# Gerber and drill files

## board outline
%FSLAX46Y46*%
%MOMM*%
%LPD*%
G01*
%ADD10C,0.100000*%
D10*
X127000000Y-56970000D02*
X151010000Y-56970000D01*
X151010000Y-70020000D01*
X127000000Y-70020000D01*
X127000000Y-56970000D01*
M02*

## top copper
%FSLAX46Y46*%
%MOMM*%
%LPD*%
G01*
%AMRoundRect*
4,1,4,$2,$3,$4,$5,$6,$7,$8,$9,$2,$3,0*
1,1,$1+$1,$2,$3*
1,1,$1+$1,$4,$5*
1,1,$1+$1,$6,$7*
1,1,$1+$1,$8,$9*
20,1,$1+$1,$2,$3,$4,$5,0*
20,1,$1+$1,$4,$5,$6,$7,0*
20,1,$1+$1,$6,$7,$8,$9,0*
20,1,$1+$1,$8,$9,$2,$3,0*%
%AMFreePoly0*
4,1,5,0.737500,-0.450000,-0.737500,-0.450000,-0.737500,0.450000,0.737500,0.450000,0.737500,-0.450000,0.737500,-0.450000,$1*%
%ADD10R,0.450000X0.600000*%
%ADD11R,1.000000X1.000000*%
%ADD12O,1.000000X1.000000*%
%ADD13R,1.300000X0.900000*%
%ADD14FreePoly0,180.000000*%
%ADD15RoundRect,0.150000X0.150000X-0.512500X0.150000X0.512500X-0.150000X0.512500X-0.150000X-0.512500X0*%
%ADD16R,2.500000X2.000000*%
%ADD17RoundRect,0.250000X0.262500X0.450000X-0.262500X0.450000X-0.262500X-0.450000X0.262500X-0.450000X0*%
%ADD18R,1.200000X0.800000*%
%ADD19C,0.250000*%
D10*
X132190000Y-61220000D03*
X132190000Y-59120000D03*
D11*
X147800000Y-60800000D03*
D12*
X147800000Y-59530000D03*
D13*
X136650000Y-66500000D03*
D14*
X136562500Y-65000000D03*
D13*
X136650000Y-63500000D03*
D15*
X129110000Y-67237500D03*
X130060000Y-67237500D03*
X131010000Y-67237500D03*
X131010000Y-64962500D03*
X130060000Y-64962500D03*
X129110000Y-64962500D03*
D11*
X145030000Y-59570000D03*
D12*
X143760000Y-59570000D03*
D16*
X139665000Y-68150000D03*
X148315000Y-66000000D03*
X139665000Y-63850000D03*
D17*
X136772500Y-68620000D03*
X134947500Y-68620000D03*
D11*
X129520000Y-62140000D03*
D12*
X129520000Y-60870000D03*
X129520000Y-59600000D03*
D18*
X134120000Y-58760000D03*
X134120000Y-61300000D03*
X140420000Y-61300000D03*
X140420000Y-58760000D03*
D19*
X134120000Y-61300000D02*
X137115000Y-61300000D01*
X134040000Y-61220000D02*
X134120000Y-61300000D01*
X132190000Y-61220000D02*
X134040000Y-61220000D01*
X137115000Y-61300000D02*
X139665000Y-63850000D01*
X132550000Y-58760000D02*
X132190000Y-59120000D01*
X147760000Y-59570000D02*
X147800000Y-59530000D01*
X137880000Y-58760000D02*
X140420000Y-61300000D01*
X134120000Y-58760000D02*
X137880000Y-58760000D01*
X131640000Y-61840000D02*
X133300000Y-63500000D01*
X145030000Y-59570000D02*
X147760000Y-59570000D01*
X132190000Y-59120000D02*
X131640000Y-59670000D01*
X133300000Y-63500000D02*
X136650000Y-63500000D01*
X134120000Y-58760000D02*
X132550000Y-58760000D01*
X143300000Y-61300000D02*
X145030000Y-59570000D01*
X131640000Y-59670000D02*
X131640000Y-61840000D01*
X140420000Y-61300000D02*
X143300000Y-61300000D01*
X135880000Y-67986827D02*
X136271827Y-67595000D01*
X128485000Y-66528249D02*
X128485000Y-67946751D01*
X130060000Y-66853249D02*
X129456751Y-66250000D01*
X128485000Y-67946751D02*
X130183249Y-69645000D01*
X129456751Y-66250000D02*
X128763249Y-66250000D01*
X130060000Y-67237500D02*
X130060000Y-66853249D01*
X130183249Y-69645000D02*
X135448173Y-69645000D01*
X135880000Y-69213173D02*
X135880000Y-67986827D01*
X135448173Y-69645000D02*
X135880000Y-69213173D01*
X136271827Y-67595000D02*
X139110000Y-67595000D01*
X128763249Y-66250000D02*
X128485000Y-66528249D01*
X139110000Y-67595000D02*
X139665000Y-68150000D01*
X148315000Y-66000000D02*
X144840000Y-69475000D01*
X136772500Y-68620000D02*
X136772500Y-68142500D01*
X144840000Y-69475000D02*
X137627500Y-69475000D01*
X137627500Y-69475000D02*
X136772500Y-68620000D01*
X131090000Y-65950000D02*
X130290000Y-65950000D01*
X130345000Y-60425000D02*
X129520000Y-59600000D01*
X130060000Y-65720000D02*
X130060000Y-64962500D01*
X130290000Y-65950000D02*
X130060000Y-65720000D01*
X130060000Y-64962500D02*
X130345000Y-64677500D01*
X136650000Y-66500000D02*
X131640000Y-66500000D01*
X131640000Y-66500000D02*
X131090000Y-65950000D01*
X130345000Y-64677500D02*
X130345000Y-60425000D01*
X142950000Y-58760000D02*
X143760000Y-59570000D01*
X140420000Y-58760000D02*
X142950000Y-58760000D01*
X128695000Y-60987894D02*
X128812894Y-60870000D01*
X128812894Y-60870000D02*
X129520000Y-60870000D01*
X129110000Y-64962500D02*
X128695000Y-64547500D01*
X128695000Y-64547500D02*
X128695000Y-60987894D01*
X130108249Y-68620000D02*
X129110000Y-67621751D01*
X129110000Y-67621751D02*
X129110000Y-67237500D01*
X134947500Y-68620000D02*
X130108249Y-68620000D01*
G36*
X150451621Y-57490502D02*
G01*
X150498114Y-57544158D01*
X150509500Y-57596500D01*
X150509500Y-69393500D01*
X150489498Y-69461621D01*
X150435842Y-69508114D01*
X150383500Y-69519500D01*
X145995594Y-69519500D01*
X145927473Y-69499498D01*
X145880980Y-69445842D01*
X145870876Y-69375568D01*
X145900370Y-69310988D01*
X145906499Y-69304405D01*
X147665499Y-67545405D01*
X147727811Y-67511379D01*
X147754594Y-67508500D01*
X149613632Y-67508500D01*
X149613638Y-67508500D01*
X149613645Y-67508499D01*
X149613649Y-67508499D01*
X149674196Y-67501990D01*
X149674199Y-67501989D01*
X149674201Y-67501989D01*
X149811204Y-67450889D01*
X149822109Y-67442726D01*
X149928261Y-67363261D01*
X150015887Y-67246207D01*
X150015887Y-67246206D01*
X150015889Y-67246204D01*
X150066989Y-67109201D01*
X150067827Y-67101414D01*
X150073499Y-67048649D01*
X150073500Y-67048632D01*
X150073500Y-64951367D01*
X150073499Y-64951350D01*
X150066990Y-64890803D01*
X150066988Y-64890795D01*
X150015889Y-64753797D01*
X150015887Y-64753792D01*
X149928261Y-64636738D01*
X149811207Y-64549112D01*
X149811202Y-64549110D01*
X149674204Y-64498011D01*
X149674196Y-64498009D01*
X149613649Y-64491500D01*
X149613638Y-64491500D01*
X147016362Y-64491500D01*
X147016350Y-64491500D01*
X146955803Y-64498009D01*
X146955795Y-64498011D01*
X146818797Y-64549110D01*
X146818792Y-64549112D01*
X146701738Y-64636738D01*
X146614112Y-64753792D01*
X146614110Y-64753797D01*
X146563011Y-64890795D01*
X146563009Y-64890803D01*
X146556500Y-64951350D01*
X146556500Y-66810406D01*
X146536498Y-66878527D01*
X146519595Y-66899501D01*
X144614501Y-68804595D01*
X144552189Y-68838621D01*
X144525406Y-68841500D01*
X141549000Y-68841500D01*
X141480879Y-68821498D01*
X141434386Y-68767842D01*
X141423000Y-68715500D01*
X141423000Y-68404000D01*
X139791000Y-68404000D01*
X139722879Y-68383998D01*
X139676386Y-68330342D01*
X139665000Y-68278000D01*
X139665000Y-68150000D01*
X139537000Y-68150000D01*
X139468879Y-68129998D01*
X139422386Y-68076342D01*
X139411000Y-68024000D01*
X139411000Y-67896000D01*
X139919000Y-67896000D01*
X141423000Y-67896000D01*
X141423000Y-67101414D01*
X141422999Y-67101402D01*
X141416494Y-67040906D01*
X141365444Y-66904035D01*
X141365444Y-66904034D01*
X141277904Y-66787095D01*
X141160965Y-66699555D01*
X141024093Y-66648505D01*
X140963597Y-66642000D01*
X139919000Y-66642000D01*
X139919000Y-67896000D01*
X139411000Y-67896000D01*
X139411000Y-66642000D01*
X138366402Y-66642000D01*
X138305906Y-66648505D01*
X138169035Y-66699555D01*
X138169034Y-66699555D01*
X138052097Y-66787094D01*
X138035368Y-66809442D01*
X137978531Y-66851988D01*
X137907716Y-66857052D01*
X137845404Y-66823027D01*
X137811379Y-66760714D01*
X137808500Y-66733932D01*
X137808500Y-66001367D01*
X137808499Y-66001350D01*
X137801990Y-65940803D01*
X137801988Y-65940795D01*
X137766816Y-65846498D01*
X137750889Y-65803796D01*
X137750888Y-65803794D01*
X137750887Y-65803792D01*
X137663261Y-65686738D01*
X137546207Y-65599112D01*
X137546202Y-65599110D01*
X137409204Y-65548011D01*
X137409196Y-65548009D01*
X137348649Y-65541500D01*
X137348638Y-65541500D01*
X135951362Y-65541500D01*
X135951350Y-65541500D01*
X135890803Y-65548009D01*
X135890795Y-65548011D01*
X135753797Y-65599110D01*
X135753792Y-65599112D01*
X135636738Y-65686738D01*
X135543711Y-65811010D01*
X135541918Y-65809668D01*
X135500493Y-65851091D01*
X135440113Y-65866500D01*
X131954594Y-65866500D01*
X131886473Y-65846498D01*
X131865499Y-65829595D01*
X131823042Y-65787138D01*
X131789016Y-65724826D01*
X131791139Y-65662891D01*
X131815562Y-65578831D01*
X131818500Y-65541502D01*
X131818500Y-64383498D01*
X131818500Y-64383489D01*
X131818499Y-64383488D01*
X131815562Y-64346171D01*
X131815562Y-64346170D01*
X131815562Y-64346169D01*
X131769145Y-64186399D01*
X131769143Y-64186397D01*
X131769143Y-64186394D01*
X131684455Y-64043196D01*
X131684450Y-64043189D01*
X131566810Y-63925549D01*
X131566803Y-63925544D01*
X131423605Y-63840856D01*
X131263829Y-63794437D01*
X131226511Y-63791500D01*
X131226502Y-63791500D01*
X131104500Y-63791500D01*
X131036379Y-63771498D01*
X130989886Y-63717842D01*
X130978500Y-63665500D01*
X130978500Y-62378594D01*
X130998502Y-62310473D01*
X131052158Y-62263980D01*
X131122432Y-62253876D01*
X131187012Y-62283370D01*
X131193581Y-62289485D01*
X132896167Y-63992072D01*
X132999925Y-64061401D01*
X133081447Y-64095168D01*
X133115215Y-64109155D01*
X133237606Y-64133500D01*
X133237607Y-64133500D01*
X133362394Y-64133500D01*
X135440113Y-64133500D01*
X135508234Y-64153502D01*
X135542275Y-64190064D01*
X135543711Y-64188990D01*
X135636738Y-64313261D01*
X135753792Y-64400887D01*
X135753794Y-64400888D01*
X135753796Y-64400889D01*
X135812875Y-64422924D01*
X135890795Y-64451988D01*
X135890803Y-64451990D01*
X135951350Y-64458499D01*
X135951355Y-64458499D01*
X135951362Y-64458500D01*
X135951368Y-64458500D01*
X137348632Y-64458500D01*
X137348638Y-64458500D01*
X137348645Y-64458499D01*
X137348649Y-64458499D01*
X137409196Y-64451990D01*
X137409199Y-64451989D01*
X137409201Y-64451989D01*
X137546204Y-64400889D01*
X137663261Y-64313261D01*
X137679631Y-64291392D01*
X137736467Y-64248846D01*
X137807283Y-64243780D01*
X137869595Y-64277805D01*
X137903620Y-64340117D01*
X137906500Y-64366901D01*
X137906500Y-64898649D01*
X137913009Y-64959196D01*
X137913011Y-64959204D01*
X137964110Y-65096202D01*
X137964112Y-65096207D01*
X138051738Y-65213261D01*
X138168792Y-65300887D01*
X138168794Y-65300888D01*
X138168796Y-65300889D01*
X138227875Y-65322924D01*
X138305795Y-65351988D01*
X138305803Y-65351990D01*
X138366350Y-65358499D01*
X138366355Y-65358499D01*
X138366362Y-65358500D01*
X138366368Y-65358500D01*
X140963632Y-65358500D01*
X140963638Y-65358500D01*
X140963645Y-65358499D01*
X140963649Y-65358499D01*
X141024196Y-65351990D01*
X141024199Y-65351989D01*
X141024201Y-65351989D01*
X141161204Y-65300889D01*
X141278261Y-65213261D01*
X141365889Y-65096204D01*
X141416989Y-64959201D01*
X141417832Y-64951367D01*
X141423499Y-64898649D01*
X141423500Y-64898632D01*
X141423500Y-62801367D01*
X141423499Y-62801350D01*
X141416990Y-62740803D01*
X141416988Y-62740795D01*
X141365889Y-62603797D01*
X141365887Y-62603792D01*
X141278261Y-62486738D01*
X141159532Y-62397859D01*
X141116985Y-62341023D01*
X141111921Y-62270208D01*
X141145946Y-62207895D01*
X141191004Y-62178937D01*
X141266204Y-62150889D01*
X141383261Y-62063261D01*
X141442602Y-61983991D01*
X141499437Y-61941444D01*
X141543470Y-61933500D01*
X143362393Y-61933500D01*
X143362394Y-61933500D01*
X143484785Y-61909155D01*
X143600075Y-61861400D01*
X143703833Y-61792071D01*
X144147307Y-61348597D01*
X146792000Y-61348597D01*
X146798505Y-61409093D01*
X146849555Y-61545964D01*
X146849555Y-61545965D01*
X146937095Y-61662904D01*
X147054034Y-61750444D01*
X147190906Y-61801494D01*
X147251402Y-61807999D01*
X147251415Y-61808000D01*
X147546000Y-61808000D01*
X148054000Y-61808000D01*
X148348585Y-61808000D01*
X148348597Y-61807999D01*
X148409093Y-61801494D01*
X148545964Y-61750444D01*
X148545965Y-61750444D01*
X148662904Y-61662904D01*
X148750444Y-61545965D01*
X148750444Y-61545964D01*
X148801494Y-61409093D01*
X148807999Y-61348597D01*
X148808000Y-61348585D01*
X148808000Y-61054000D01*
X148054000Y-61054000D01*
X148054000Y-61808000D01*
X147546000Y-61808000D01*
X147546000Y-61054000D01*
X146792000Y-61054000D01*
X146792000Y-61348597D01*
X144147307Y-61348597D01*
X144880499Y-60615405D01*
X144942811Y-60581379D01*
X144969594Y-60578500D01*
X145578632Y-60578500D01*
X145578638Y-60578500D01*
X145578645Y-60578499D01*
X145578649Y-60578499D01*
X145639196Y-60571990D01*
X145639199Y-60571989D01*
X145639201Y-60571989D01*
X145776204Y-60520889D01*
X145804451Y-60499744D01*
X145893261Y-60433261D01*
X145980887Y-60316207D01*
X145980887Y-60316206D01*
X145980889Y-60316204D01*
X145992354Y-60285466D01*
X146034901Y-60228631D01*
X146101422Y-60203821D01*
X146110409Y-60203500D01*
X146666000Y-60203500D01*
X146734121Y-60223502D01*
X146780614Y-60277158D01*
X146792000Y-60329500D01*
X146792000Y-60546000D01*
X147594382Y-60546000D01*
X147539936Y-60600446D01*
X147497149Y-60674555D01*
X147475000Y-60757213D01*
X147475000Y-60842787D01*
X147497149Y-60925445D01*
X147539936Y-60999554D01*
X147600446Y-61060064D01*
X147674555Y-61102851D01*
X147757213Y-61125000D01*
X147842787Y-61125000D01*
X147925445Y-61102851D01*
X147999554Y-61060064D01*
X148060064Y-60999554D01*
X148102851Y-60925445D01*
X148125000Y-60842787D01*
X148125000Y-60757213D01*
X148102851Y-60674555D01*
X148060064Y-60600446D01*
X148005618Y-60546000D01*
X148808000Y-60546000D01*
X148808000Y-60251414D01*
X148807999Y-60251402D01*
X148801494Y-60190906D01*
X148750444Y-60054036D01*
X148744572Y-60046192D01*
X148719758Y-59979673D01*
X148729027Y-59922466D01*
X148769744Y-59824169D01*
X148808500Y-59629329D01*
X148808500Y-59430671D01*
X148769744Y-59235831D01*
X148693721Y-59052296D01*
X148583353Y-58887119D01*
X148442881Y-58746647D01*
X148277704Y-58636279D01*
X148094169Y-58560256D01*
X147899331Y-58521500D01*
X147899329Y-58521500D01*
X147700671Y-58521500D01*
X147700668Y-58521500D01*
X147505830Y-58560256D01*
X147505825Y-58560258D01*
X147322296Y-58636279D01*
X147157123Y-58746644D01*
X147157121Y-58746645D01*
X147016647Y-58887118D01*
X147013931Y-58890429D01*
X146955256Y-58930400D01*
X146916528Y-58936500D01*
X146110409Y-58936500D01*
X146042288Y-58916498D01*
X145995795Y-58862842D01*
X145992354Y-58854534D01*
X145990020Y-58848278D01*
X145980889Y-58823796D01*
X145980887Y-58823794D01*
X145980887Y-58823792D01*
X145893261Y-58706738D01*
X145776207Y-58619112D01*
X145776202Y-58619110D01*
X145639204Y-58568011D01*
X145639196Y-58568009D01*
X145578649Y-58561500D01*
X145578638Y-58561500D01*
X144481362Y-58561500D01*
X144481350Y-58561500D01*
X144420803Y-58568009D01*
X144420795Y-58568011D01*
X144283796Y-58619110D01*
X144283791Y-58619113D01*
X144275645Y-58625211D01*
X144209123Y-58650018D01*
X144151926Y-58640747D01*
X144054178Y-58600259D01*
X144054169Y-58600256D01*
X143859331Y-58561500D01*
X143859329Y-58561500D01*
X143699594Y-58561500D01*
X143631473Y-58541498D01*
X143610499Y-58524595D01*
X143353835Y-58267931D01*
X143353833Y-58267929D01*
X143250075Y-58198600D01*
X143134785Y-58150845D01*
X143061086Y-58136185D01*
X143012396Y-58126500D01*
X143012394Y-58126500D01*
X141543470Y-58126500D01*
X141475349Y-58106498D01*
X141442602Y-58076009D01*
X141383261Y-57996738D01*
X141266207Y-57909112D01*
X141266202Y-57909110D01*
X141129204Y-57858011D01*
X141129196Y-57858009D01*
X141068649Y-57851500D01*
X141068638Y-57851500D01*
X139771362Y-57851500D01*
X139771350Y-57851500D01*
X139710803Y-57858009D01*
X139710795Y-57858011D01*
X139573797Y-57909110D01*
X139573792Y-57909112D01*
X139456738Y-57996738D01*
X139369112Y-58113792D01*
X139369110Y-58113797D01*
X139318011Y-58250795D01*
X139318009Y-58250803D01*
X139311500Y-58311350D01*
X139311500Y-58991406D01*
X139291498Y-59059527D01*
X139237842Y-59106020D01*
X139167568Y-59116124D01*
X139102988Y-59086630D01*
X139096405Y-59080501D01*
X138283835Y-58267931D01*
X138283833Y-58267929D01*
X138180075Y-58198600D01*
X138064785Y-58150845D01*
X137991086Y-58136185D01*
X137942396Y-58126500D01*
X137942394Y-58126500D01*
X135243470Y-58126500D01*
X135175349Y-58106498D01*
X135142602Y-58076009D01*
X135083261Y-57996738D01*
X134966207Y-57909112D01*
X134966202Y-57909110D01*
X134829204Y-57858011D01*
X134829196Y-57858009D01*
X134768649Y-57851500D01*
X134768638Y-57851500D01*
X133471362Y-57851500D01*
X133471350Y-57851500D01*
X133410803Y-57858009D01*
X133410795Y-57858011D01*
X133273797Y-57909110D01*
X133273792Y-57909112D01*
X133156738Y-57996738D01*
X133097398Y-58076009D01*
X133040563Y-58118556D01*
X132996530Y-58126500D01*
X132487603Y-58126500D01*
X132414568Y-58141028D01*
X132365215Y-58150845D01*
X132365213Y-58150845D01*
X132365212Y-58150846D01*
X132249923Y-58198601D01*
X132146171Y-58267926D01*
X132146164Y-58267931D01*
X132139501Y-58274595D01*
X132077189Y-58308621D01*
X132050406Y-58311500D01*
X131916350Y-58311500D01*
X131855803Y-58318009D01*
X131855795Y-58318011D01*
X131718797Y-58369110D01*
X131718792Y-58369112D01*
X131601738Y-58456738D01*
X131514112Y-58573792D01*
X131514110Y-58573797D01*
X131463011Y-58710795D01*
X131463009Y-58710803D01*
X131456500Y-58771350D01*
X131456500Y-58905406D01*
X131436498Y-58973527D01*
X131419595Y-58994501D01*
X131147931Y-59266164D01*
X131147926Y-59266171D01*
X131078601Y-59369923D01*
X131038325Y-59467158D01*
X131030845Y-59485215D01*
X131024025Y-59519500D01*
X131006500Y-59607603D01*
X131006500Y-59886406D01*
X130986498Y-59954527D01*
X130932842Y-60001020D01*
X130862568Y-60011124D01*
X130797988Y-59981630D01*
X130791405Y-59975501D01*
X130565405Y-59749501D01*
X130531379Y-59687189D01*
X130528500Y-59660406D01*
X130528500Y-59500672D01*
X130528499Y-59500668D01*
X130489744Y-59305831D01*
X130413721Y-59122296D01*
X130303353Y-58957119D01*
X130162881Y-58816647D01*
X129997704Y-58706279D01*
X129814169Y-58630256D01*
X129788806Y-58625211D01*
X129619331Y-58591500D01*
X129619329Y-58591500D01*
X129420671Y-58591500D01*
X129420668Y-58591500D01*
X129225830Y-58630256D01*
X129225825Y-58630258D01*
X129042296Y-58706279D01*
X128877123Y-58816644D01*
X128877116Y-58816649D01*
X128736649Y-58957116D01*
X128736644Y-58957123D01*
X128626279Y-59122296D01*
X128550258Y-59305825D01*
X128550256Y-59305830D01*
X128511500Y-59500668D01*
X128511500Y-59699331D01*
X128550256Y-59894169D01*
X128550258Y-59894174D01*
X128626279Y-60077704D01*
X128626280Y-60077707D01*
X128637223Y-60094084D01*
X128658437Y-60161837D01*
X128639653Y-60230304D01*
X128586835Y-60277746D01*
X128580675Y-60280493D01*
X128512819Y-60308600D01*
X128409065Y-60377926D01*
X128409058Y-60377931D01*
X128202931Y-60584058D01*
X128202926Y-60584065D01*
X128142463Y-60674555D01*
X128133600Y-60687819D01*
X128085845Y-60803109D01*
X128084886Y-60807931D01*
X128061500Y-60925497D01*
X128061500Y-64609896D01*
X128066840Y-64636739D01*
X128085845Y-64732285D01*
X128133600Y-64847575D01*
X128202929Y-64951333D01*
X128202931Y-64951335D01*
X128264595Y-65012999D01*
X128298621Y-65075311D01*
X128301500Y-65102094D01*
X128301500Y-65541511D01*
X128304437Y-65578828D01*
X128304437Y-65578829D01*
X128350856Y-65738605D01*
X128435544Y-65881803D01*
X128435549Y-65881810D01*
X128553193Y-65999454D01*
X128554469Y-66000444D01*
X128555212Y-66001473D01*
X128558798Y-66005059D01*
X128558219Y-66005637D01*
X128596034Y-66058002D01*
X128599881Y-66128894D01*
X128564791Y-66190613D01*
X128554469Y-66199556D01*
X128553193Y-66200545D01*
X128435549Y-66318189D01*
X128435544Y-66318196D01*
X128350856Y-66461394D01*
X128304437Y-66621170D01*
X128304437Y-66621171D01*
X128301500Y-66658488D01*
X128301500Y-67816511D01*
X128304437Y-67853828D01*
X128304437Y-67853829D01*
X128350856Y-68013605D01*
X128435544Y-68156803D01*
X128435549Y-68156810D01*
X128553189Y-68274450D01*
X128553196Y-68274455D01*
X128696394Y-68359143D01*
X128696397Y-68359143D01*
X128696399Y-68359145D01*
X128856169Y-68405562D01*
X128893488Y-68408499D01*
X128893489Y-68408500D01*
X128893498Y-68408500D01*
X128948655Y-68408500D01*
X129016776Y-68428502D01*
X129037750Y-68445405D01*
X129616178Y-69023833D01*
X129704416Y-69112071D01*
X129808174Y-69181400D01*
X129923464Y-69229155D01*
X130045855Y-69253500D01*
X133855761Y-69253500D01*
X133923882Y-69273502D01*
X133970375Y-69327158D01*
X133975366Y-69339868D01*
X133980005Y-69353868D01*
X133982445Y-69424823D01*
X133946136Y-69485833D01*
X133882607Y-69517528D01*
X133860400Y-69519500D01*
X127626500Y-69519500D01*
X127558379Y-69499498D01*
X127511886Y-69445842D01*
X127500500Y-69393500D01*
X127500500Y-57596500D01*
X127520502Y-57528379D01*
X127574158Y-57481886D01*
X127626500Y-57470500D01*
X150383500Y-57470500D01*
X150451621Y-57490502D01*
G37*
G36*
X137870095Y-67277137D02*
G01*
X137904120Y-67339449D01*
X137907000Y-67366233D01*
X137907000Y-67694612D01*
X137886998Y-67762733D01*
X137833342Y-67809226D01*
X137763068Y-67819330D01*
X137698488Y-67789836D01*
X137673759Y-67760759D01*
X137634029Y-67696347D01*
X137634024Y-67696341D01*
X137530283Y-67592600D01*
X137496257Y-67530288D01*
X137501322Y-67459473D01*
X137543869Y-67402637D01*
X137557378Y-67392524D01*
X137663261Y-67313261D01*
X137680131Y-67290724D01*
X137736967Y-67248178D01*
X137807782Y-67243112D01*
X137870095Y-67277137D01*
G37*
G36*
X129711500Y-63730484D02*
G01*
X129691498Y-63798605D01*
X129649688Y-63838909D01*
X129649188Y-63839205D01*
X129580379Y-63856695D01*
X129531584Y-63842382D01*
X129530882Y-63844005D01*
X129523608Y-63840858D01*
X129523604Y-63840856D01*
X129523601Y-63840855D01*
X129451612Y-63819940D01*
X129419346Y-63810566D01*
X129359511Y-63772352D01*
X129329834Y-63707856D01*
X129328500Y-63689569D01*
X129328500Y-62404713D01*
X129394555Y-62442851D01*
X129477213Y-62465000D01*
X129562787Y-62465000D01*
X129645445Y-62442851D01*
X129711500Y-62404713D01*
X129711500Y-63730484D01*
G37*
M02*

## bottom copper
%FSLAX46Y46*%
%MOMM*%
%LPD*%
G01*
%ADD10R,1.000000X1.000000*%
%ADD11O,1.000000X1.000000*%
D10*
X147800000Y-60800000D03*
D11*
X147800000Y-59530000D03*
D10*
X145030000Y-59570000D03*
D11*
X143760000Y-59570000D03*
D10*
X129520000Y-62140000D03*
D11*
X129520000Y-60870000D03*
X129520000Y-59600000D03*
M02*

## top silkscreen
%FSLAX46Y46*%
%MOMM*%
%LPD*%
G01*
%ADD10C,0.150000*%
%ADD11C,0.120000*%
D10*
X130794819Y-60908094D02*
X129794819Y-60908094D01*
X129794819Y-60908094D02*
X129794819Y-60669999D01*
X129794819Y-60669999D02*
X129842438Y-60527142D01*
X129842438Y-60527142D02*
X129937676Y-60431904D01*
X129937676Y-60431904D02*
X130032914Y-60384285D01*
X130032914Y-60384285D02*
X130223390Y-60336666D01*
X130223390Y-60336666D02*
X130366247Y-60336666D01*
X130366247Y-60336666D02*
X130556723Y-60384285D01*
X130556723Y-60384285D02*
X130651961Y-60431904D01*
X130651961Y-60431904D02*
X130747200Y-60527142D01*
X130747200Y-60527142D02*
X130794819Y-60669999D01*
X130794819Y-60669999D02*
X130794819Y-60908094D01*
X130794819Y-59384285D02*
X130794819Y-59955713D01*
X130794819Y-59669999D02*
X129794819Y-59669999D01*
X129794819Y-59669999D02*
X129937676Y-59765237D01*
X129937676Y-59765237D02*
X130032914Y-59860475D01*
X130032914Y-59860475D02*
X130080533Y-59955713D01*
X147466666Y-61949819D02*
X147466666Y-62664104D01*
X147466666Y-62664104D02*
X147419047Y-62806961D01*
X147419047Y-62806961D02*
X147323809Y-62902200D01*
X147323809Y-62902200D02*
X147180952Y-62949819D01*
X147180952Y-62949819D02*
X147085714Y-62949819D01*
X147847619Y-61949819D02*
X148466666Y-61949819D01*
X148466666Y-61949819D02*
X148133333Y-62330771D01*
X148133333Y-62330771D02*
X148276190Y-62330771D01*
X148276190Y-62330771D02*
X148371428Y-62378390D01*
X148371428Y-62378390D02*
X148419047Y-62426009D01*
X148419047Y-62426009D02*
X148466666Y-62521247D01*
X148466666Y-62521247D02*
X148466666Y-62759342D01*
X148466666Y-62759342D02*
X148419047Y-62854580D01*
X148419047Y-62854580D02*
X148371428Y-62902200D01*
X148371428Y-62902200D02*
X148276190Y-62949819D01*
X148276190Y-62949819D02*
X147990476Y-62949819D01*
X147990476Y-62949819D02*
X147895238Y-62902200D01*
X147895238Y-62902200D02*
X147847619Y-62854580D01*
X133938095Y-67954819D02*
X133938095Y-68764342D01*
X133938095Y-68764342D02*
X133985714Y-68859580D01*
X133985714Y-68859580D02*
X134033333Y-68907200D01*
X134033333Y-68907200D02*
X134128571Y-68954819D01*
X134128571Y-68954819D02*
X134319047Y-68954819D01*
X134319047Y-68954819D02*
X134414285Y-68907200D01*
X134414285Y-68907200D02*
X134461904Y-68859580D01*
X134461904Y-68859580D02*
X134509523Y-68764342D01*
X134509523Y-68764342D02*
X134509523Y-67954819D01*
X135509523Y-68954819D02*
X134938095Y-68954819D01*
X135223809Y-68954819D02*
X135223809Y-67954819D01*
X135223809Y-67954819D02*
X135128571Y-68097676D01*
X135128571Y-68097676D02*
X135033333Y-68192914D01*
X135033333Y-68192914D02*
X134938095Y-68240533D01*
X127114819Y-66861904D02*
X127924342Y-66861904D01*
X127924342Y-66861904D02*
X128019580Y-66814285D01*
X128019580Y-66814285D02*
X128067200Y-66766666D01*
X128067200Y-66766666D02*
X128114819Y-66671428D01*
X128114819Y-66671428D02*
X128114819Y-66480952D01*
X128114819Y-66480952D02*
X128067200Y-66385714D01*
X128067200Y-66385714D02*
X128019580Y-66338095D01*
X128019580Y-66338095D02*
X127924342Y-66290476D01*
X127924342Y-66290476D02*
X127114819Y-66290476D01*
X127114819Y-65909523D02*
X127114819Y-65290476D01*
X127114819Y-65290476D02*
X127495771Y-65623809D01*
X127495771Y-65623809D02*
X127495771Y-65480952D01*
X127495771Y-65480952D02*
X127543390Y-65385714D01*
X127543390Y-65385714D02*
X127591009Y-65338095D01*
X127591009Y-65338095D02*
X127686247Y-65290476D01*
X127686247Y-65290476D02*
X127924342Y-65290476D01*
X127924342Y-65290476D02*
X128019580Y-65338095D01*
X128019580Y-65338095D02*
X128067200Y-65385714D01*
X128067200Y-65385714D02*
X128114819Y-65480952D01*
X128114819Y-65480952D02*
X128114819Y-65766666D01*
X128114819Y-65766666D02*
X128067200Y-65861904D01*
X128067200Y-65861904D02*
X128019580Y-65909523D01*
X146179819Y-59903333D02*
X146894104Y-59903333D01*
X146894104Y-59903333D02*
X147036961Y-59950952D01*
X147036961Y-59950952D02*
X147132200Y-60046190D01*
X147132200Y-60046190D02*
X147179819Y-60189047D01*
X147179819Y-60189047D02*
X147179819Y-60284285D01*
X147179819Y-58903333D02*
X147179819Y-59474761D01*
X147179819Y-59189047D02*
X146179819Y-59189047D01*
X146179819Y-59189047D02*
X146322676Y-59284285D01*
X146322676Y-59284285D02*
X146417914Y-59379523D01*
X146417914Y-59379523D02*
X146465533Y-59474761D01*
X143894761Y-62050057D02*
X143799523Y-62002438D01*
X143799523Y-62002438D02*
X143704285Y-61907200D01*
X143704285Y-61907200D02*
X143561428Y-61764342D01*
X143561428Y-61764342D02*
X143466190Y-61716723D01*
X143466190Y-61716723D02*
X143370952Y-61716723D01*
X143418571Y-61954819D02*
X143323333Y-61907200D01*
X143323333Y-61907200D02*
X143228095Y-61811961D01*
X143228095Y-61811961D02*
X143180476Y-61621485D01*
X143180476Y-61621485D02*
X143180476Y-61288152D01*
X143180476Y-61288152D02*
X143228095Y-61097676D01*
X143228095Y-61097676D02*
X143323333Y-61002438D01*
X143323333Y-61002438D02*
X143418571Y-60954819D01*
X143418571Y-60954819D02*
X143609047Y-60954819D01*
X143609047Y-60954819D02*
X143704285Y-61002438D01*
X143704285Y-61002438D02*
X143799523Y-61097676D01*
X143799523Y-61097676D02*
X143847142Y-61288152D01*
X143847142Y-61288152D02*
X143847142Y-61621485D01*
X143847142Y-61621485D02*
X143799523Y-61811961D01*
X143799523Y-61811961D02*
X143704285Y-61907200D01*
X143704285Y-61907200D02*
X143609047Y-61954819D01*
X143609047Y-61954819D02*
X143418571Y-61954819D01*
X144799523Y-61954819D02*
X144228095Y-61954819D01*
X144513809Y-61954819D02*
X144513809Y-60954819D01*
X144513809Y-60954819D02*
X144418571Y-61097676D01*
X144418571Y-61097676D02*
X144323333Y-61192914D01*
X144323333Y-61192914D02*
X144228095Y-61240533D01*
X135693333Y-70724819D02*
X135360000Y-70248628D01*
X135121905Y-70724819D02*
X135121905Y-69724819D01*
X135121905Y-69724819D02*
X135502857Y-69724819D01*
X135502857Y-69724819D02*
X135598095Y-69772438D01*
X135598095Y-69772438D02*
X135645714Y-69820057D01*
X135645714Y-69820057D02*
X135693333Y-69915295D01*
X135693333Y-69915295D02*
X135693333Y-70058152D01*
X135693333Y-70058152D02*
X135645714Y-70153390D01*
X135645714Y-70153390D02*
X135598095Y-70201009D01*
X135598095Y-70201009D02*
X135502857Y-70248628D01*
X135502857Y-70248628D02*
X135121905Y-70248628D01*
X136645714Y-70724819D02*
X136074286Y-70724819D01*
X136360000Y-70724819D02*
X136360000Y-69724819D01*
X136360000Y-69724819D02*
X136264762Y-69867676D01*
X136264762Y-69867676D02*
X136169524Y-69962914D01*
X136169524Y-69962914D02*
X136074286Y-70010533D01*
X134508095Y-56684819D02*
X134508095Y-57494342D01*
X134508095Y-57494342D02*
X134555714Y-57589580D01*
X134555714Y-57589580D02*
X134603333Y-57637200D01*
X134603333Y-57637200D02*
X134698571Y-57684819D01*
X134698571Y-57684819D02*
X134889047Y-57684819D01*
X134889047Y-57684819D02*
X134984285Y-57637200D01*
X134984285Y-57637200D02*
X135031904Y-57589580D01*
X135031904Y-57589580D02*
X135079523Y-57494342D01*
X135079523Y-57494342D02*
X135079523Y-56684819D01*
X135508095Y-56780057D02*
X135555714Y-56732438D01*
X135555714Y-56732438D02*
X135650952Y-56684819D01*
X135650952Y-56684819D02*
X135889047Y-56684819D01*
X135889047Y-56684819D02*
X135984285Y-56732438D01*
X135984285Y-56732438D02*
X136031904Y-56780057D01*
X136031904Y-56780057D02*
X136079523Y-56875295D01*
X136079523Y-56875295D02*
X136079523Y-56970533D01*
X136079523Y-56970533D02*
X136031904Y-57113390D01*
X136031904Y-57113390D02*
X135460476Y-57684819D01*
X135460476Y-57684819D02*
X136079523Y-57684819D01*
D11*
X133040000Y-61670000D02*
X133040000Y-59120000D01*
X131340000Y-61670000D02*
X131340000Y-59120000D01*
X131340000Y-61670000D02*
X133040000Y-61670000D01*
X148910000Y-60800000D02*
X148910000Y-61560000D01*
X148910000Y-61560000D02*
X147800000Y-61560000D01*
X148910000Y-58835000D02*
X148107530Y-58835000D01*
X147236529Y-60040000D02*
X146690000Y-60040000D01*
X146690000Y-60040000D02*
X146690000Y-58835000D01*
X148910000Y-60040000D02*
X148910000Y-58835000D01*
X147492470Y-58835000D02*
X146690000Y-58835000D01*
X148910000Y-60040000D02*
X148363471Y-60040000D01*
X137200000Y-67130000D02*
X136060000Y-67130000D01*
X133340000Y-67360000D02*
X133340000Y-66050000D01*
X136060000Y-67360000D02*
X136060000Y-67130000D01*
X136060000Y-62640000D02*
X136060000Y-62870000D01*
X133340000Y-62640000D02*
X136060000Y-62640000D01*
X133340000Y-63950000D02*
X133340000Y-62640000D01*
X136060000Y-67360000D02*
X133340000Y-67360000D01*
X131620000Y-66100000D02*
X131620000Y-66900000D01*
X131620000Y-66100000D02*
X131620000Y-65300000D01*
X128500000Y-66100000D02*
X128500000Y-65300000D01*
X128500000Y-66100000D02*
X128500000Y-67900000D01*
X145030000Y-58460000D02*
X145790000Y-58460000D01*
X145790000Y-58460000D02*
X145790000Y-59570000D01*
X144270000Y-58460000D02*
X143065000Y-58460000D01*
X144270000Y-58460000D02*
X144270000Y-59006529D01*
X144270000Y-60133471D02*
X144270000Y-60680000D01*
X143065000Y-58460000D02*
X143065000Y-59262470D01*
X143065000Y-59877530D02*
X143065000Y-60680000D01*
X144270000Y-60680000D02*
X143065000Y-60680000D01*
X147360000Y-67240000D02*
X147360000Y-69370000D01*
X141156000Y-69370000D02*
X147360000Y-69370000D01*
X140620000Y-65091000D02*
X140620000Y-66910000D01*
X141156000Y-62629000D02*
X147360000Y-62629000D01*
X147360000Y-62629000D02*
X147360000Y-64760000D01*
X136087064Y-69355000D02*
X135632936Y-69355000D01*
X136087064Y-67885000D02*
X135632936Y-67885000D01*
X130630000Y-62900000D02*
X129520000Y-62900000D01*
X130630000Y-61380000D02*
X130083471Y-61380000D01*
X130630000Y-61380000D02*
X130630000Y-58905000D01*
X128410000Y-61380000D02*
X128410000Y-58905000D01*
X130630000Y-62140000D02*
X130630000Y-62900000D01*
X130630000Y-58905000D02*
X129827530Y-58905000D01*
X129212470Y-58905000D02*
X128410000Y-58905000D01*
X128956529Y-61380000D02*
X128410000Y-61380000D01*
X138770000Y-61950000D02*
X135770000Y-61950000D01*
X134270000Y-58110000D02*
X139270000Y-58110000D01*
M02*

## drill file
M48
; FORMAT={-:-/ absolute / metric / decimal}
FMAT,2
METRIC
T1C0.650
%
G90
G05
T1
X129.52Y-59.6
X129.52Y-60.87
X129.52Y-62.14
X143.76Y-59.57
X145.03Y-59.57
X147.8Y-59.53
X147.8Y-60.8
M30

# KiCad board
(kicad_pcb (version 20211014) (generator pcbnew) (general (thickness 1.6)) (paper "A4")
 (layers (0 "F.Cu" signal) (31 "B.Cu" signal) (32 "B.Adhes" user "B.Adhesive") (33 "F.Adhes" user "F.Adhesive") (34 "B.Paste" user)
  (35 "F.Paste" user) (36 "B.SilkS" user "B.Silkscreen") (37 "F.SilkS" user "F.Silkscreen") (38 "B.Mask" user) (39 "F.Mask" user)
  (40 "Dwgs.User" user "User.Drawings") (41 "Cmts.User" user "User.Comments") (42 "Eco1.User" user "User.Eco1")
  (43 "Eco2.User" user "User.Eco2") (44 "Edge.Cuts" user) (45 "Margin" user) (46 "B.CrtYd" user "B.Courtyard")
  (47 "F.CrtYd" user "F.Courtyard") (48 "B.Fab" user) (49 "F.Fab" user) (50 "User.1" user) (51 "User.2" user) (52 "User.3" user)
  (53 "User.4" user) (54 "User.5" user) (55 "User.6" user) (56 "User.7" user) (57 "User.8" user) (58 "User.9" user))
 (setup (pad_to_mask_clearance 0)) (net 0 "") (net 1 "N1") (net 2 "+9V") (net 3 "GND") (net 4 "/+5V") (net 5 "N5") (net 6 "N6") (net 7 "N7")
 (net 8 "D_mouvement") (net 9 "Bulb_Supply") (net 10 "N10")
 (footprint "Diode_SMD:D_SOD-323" (layer "F.Cu") (at 132.19 60.17 90)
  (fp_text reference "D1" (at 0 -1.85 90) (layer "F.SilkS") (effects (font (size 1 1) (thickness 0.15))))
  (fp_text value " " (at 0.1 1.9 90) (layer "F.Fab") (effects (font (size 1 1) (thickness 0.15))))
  (fp_line (start -1.5 0.85) (end 1.05 0.85) (layer "F.SilkS") (width 0.12))
  (fp_line (start -1.5 -0.85) (end 1.05 -0.85) (layer "F.SilkS") (width 0.12))
  (fp_line (start -1.5 -0.85) (end -1.5 0.85) (layer "F.SilkS") (width 0.12))
  (pad "1" smd rect (at -1.05 0 90) (size 0.6 0.45) (layers "F.Cu" "F.Paste" "F.Mask") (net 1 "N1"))
  (pad "2" smd rect (at 1.05 0 90) (size 0.6 0.45) (layers "F.Cu" "F.Paste" "F.Mask") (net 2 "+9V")))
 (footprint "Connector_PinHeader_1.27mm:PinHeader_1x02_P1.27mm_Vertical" (layer "F.Cu") (at 147.8 60.8 180)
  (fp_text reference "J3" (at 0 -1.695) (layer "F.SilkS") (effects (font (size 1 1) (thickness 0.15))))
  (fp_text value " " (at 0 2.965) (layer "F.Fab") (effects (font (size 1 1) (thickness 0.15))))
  (fp_line (start -1.11 0) (end -1.11 -0.76) (layer "F.SilkS") (width 0.12))
  (fp_line (start -1.11 -0.76) (end 0 -0.76) (layer "F.SilkS") (width 0.12))
  (fp_line (start -1.11 1.965) (end -0.30753 1.965) (layer "F.SilkS") (width 0.12))
  (fp_line (start 0.563471 0.76) (end 1.11 0.76) (layer "F.SilkS") (width 0.12))
  (fp_line (start 1.11 0.76) (end 1.11 1.965) (layer "F.SilkS") (width 0.12))
  (fp_line (start -1.11 0.76) (end -1.11 1.965) (layer "F.SilkS") (width 0.12))
  (fp_line (start 0.30753 1.965) (end 1.11 1.965) (layer "F.SilkS") (width 0.12))
  (fp_line (start -1.11 0.76) (end -0.563471 0.76) (layer "F.SilkS") (width 0.12))
  (pad "1" thru_hole rect (at 0 0 180) (size 1 1) (drill 0.65) (layers *.Cu *.Mask) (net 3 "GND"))
  (pad "2" thru_hole oval (at 0 1.27 180) (size 1 1) (drill 0.65) (layers *.Cu *.Mask) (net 2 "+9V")))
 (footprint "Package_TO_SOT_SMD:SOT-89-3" (layer "F.Cu") (at 135 65 180)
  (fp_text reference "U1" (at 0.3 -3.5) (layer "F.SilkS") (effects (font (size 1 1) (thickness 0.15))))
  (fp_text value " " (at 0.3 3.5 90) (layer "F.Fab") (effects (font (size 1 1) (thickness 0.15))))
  (fp_line (start -2.2 -2.13) (end -1.06 -2.13) (layer "F.SilkS") (width 0.12))
  (fp_line (start 1.66 -2.36) (end 1.66 -1.05) (layer "F.SilkS") (width 0.12))
  (fp_line (start -1.06 -2.36) (end -1.06 -2.13) (layer "F.SilkS") (width 0.12))
  (fp_line (start -1.06 2.36) (end -1.06 2.13) (layer "F.SilkS") (width 0.12))
  (fp_line (start 1.66 2.36) (end -1.06 2.36) (layer "F.SilkS") (width 0.12))
  (fp_line (start 1.66 1.05) (end 1.66 2.36) (layer "F.SilkS") (width 0.12))
  (fp_line (start -1.06 -2.36) (end 1.66 -2.36) (layer "F.SilkS") (width 0.12))
  (pad "1" smd rect (at -1.65 -1.5 180) (size 1.3 0.9) (layers "F.Cu" "F.Paste" "F.Mask") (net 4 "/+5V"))
  (pad "2" smd custom (at -1.5625 0 180) (size 1.475 0.9) (layers "F.Cu" "F.Paste" "F.Mask") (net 3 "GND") (zone_connect 2)
   (options (clearance outline) (anchor rect)) (primitives))
  (pad "3" smd rect (at -1.65 1.5 180) (size 1.3 0.9) (layers "F.Cu" "F.Paste" "F.Mask") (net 2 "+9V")))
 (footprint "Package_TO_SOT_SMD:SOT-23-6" (layer "F.Cu") (at 130.06 66.1 90)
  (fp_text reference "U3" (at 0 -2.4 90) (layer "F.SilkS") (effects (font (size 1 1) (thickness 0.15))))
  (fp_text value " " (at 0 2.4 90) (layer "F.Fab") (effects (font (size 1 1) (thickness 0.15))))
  (fp_line (start 0 1.56) (end -0.8 1.56) (layer "F.SilkS") (width 0.12))
  (fp_line (start 0 1.56) (end 0.8 1.56) (layer "F.SilkS") (width 0.12))
  (fp_line (start 0 -1.56) (end 0.8 -1.56) (layer "F.SilkS") (width 0.12))
  (fp_line (start 0 -1.56) (end -1.8 -1.56) (layer "F.SilkS") (width 0.12))
  (pad "1" smd roundrect (at -1.1375 -0.95 90) (size 1.325 0.6) (layers "F.Cu" "F.Paste" "F.Mask") (roundrect_rratio 0.25) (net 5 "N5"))
  (pad "2" smd roundrect (at -1.1375 0 90) (size 1.325 0.6) (layers "F.Cu" "F.Paste" "F.Mask") (roundrect_rratio 0.25) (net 3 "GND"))
  (pad "3" smd roundrect (at -1.1375 0.95 90) (size 1.325 0.6) (layers "F.Cu" "F.Paste" "F.Mask") (roundrect_rratio 0.25) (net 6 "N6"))
  (pad "4" smd roundrect (at 1.1375 0.95 90) (size 1.325 0.6) (layers "F.Cu" "F.Paste" "F.Mask") (roundrect_rratio 0.25) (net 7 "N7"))
  (pad "5" smd roundrect (at 1.1375 0 90) (size 1.325 0.6) (layers "F.Cu" "F.Paste" "F.Mask") (roundrect_rratio 0.25) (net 4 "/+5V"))
  (pad "6" smd roundrect (at 1.1375 -0.95 90) (size 1.325 0.6) (layers "F.Cu" "F.Paste" "F.Mask") (roundrect_rratio 0.25)
   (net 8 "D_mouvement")))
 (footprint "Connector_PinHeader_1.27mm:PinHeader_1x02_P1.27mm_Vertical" (layer "F.Cu") (at 145.03 59.57 -90)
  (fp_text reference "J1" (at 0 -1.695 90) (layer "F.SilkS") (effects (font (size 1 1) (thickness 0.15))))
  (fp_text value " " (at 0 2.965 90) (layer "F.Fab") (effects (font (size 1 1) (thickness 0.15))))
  (fp_line (start -1.11 0) (end -1.11 -0.76) (layer "F.SilkS") (width 0.12))
  (fp_line (start -1.11 -0.76) (end 0 -0.76) (layer "F.SilkS") (width 0.12))
  (fp_line (start -1.11 0.76) (end -1.11 1.965) (layer "F.SilkS") (width 0.12))
  (fp_line (start -1.11 0.76) (end -0.563471 0.76) (layer "F.SilkS") (width 0.12))
  (fp_line (start 0.563471 0.76) (end 1.11 0.76) (layer "F.SilkS") (width 0.12))
  (fp_line (start -1.11 1.965) (end -0.30753 1.965) (layer "F.SilkS") (width 0.12))
  (fp_line (start 0.30753 1.965) (end 1.11 1.965) (layer "F.SilkS") (width 0.12))
  (fp_line (start 1.11 0.76) (end 1.11 1.965) (layer "F.SilkS") (width 0.12))
  (pad "1" thru_hole rect (at 0 0 270) (size 1 1) (drill 0.65) (layers *.Cu *.Mask) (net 2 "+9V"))
  (pad "2" thru_hole oval (at 0 1.27 270) (size 1 1) (drill 0.65) (layers *.Cu *.Mask) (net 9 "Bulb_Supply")))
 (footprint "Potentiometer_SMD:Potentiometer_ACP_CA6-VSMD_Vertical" (layer "F.Cu") (at 143.99 66)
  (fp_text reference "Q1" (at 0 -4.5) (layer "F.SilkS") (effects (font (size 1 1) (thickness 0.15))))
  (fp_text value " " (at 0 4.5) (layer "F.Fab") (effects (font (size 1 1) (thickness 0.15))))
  (fp_line (start 3.37 1.24) (end 3.37 3.37) (layer "F.SilkS") (width 0.12))
  (fp_line (start -2.834 3.37) (end 3.37 3.37) (layer "F.SilkS") (width 0.12))
  (fp_line (start -3.37 -0.909) (end -3.37 0.91) (layer "F.SilkS") (width 0.12))
  (fp_line (start -2.834 -3.371) (end 3.37 -3.371) (layer "F.SilkS") (width 0.12))
  (fp_line (start 3.37 -3.371) (end 3.37 -1.24) (layer "F.SilkS") (width 0.12))
  (pad "1" smd rect (at -4.325 2.15) (size 2.5 2) (layers "F.Cu" "F.Paste" "F.Mask") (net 3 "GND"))
  (pad "2" smd rect (at 4.325 0) (size 2.5 2) (layers "F.Cu" "F.Paste" "F.Mask") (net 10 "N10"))
  (pad "3" smd rect (at -4.325 -2.15) (size 2.5 2) (layers "F.Cu" "F.Paste" "F.Mask") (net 1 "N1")))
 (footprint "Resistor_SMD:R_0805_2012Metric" (layer "F.Cu") (at 135.86 68.62 180)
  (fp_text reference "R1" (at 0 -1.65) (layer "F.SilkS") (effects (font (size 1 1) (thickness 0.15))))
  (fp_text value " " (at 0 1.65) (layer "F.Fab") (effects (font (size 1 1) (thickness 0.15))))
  (fp_line (start -0.227064 -0.735) (end 0.227064 -0.735) (layer "F.SilkS") (width 0.12))
  (fp_line (start -0.227064 0.735) (end 0.227064 0.735) (layer "F.SilkS") (width 0.12))
  (pad "1" smd roundrect (at -0.9125 0 180) (size 1.025 1.4) (layers "F.Cu" "F.Paste" "F.Mask") (roundrect_rratio 0.243902) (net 10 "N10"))
  (pad "2" smd roundrect (at 0.9125 0 180) (size 1.025 1.4) (layers "F.Cu" "F.Paste" "F.Mask") (roundrect_rratio 0.243902) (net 5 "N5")))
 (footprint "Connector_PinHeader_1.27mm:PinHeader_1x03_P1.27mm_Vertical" (layer "F.Cu") (at 129.52 62.14 180)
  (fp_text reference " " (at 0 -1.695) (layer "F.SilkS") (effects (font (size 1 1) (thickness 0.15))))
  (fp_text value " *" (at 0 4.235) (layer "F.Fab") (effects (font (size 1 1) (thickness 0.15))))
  (fp_line (start -1.11 -0.76) (end 0 -0.76) (layer "F.SilkS") (width 0.12))
  (fp_line (start -1.11 0.76) (end -0.563471 0.76) (layer "F.SilkS") (width 0.12))
  (fp_line (start -1.11 0.76) (end -1.11 3.235) (layer "F.SilkS") (width 0.12))
  (fp_line (start 1.11 0.76) (end 1.11 3.235) (layer "F.SilkS") (width 0.12))
  (fp_line (start -1.11 0) (end -1.11 -0.76) (layer "F.SilkS") (width 0.12))
  (fp_line (start -1.11 3.235) (end -0.30753 3.235) (layer "F.SilkS") (width 0.12))
  (fp_line (start 0.30753 3.235) (end 1.11 3.235) (layer "F.SilkS") (width 0.12))
  (fp_line (start 0.563471 0.76) (end 1.11 0.76) (layer "F.SilkS") (width 0.12))
  (pad "1" thru_hole rect (at 0 0 180) (size 1 1) (drill 0.65) (layers *.Cu *.Mask) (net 3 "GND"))
  (pad "2" thru_hole oval (at 0 1.27 180) (size 1 1) (drill 0.65) (layers *.Cu *.Mask) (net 8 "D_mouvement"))
  (pad "3" thru_hole oval (at 0 2.54 180) (size 1 1) (drill 0.65) (layers *.Cu *.Mask) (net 4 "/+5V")))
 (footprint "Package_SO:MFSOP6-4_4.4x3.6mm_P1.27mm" (layer "F.Cu") (at 137.27 60.03)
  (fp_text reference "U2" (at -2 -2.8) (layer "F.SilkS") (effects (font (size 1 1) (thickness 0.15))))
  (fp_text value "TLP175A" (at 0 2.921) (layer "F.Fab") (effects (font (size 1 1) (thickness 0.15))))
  (fp_line (start 1.5 1.92) (end -1.5 1.92) (layer "F.SilkS") (width 0.12))
  (fp_line (start -3 -1.92) (end 2 -1.92) (layer "F.SilkS") (width 0.12))
  (pad "1" smd rect (at -3.15 -1.27) (size 1.2 0.8) (layers "F.Cu" "F.Paste" "F.Mask") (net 2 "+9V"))
  (pad "3" smd rect (at -3.15 1.27) (size 1.2 0.8) (layers "F.Cu" "F.Paste" "F.Mask") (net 1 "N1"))
  (pad "4" smd rect (at 3.15 1.27) (size 1.2 0.8) (layers "F.Cu" "F.Paste" "F.Mask") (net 2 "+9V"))
  (pad "6" smd rect (at 3.15 -1.27) (size 1.2 0.8) (layers "F.Cu" "F.Paste" "F.Mask") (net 9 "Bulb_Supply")))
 (gr_rect (start 127 56.97) (end 151.01 70.02) (layer "Edge.Cuts") (width 0.1) (fill none))
 (segment (start 134.12 61.3) (end 137.115 61.3) (width 0.25) (layer "F.Cu") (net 1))
 (segment (start 134.04 61.22) (end 134.12 61.3) (width 0.25) (layer "F.Cu") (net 1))
 (segment (start 132.19 61.22) (end 134.04 61.22) (width 0.25) (layer "F.Cu") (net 1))
 (segment (start 137.115 61.3) (end 139.665 63.85) (width 0.25) (layer "F.Cu") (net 1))
 (segment (start 132.55 58.76) (end 132.19 59.12) (width 0.25) (layer "F.Cu") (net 2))
 (segment (start 147.76 59.57) (end 147.8 59.53) (width 0.25) (layer "F.Cu") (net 2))
 (segment (start 137.88 58.76) (end 140.42 61.3) (width 0.25) (layer "F.Cu") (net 2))
 (segment (start 134.12 58.76) (end 137.88 58.76) (width 0.25) (layer "F.Cu") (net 2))
 (segment (start 131.64 61.84) (end 133.3 63.5) (width 0.25) (layer "F.Cu") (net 2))
 (segment (start 145.03 59.57) (end 147.76 59.57) (width 0.25) (layer "F.Cu") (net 2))
 (segment (start 132.19 59.12) (end 131.64 59.67) (width 0.25) (layer "F.Cu") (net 2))
 (segment (start 133.3 63.5) (end 136.65 63.5) (width 0.25) (layer "F.Cu") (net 2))
 (segment (start 134.12 58.76) (end 132.55 58.76) (width 0.25) (layer "F.Cu") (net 2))
 (segment (start 143.3 61.3) (end 145.03 59.57) (width 0.25) (layer "F.Cu") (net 2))
 (segment (start 131.64 59.67) (end 131.64 61.84) (width 0.25) (layer "F.Cu") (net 2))
 (segment (start 140.42 61.3) (end 143.3 61.3) (width 0.25) (layer "F.Cu") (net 2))
 (segment (start 135.88 67.986827) (end 136.271827 67.595) (width 0.25) (layer "F.Cu") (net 3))
 (segment (start 128.485 66.528249) (end 128.485 67.946751) (width 0.25) (layer "F.Cu") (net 3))
 (segment (start 130.06 66.853249) (end 129.456751 66.25) (width 0.25) (layer "F.Cu") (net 3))
 (segment (start 128.485 67.946751) (end 130.183249 69.645) (width 0.25) (layer "F.Cu") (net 3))
 (segment (start 129.456751 66.25) (end 128.763249 66.25) (width 0.25) (layer "F.Cu") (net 3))
 (segment (start 130.06 67.2375) (end 130.06 66.853249) (width 0.25) (layer "F.Cu") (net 3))
 (segment (start 130.183249 69.645) (end 135.448173 69.645) (width 0.25) (layer "F.Cu") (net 3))
 (segment (start 135.88 69.213173) (end 135.88 67.986827) (width 0.25) (layer "F.Cu") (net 3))
 (segment (start 135.448173 69.645) (end 135.88 69.213173) (width 0.25) (layer "F.Cu") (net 3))
 (segment (start 136.271827 67.595) (end 139.11 67.595) (width 0.25) (layer "F.Cu") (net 3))
 (segment (start 128.763249 66.25) (end 128.485 66.528249) (width 0.25) (layer "F.Cu") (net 3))
 (segment (start 139.11 67.595) (end 139.665 68.15) (width 0.25) (layer "F.Cu") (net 3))
 (segment (start 148.315 66) (end 144.84 69.475) (width 0.25) (layer "F.Cu") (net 10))
 (segment (start 136.7725 68.62) (end 136.7725 68.1425) (width 0.25) (layer "F.Cu") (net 10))
 (segment (start 144.84 69.475) (end 137.6275 69.475) (width 0.25) (layer "F.Cu") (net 10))
 (segment (start 137.6275 69.475) (end 136.7725 68.62) (width 0.25) (layer "F.Cu") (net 10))
 (segment (start 131.09 65.95) (end 130.29 65.95) (width 0.25) (layer "F.Cu") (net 4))
 (segment (start 130.345 60.425) (end 129.52 59.6) (width 0.25) (layer "F.Cu") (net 4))
 (segment (start 130.06 65.72) (end 130.06 64.9625) (width 0.25) (layer "F.Cu") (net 4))
 (segment (start 130.29 65.95) (end 130.06 65.72) (width 0.25) (layer "F.Cu") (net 4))
 (segment (start 130.06 64.9625) (end 130.345 64.6775) (width 0.25) (layer "F.Cu") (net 4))
 (segment (start 136.65 66.5) (end 131.64 66.5) (width 0.25) (layer "F.Cu") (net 4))
 (segment (start 131.64 66.5) (end 131.09 65.95) (width 0.25) (layer "F.Cu") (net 4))
 (segment (start 130.345 64.6775) (end 130.345 60.425) (width 0.25) (layer "F.Cu") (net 4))
 (segment (start 142.95 58.76) (end 143.76 59.57) (width 0.25) (layer "F.Cu") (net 9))
 (segment (start 140.42 58.76) (end 142.95 58.76) (width 0.25) (layer "F.Cu") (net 9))
 (segment (start 128.695 60.987894) (end 128.812894 60.87) (width 0.25) (layer "F.Cu") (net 8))
 (segment (start 128.812894 60.87) (end 129.52 60.87) (width 0.25) (layer "F.Cu") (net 8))
 (segment (start 129.11 64.9625) (end 128.695 64.5475) (width 0.25) (layer "F.Cu") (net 8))
 (segment (start 128.695 64.5475) (end 128.695 60.987894) (width 0.25) (layer "F.Cu") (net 8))
 (segment (start 130.108249 68.62) (end 129.11 67.621751) (width 0.25) (layer "F.Cu") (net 5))
 (segment (start 129.11 67.621751) (end 129.11 67.2375) (width 0.25) (layer "F.Cu") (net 5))
 (segment (start 134.9475 68.62) (end 130.108249 68.62) (width 0.25) (layer "F.Cu") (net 5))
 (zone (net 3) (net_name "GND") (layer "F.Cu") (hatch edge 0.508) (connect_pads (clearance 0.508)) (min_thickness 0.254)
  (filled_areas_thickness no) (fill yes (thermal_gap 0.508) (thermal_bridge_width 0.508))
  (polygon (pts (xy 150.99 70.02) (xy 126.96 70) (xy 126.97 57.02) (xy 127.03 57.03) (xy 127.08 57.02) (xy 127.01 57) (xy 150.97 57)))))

